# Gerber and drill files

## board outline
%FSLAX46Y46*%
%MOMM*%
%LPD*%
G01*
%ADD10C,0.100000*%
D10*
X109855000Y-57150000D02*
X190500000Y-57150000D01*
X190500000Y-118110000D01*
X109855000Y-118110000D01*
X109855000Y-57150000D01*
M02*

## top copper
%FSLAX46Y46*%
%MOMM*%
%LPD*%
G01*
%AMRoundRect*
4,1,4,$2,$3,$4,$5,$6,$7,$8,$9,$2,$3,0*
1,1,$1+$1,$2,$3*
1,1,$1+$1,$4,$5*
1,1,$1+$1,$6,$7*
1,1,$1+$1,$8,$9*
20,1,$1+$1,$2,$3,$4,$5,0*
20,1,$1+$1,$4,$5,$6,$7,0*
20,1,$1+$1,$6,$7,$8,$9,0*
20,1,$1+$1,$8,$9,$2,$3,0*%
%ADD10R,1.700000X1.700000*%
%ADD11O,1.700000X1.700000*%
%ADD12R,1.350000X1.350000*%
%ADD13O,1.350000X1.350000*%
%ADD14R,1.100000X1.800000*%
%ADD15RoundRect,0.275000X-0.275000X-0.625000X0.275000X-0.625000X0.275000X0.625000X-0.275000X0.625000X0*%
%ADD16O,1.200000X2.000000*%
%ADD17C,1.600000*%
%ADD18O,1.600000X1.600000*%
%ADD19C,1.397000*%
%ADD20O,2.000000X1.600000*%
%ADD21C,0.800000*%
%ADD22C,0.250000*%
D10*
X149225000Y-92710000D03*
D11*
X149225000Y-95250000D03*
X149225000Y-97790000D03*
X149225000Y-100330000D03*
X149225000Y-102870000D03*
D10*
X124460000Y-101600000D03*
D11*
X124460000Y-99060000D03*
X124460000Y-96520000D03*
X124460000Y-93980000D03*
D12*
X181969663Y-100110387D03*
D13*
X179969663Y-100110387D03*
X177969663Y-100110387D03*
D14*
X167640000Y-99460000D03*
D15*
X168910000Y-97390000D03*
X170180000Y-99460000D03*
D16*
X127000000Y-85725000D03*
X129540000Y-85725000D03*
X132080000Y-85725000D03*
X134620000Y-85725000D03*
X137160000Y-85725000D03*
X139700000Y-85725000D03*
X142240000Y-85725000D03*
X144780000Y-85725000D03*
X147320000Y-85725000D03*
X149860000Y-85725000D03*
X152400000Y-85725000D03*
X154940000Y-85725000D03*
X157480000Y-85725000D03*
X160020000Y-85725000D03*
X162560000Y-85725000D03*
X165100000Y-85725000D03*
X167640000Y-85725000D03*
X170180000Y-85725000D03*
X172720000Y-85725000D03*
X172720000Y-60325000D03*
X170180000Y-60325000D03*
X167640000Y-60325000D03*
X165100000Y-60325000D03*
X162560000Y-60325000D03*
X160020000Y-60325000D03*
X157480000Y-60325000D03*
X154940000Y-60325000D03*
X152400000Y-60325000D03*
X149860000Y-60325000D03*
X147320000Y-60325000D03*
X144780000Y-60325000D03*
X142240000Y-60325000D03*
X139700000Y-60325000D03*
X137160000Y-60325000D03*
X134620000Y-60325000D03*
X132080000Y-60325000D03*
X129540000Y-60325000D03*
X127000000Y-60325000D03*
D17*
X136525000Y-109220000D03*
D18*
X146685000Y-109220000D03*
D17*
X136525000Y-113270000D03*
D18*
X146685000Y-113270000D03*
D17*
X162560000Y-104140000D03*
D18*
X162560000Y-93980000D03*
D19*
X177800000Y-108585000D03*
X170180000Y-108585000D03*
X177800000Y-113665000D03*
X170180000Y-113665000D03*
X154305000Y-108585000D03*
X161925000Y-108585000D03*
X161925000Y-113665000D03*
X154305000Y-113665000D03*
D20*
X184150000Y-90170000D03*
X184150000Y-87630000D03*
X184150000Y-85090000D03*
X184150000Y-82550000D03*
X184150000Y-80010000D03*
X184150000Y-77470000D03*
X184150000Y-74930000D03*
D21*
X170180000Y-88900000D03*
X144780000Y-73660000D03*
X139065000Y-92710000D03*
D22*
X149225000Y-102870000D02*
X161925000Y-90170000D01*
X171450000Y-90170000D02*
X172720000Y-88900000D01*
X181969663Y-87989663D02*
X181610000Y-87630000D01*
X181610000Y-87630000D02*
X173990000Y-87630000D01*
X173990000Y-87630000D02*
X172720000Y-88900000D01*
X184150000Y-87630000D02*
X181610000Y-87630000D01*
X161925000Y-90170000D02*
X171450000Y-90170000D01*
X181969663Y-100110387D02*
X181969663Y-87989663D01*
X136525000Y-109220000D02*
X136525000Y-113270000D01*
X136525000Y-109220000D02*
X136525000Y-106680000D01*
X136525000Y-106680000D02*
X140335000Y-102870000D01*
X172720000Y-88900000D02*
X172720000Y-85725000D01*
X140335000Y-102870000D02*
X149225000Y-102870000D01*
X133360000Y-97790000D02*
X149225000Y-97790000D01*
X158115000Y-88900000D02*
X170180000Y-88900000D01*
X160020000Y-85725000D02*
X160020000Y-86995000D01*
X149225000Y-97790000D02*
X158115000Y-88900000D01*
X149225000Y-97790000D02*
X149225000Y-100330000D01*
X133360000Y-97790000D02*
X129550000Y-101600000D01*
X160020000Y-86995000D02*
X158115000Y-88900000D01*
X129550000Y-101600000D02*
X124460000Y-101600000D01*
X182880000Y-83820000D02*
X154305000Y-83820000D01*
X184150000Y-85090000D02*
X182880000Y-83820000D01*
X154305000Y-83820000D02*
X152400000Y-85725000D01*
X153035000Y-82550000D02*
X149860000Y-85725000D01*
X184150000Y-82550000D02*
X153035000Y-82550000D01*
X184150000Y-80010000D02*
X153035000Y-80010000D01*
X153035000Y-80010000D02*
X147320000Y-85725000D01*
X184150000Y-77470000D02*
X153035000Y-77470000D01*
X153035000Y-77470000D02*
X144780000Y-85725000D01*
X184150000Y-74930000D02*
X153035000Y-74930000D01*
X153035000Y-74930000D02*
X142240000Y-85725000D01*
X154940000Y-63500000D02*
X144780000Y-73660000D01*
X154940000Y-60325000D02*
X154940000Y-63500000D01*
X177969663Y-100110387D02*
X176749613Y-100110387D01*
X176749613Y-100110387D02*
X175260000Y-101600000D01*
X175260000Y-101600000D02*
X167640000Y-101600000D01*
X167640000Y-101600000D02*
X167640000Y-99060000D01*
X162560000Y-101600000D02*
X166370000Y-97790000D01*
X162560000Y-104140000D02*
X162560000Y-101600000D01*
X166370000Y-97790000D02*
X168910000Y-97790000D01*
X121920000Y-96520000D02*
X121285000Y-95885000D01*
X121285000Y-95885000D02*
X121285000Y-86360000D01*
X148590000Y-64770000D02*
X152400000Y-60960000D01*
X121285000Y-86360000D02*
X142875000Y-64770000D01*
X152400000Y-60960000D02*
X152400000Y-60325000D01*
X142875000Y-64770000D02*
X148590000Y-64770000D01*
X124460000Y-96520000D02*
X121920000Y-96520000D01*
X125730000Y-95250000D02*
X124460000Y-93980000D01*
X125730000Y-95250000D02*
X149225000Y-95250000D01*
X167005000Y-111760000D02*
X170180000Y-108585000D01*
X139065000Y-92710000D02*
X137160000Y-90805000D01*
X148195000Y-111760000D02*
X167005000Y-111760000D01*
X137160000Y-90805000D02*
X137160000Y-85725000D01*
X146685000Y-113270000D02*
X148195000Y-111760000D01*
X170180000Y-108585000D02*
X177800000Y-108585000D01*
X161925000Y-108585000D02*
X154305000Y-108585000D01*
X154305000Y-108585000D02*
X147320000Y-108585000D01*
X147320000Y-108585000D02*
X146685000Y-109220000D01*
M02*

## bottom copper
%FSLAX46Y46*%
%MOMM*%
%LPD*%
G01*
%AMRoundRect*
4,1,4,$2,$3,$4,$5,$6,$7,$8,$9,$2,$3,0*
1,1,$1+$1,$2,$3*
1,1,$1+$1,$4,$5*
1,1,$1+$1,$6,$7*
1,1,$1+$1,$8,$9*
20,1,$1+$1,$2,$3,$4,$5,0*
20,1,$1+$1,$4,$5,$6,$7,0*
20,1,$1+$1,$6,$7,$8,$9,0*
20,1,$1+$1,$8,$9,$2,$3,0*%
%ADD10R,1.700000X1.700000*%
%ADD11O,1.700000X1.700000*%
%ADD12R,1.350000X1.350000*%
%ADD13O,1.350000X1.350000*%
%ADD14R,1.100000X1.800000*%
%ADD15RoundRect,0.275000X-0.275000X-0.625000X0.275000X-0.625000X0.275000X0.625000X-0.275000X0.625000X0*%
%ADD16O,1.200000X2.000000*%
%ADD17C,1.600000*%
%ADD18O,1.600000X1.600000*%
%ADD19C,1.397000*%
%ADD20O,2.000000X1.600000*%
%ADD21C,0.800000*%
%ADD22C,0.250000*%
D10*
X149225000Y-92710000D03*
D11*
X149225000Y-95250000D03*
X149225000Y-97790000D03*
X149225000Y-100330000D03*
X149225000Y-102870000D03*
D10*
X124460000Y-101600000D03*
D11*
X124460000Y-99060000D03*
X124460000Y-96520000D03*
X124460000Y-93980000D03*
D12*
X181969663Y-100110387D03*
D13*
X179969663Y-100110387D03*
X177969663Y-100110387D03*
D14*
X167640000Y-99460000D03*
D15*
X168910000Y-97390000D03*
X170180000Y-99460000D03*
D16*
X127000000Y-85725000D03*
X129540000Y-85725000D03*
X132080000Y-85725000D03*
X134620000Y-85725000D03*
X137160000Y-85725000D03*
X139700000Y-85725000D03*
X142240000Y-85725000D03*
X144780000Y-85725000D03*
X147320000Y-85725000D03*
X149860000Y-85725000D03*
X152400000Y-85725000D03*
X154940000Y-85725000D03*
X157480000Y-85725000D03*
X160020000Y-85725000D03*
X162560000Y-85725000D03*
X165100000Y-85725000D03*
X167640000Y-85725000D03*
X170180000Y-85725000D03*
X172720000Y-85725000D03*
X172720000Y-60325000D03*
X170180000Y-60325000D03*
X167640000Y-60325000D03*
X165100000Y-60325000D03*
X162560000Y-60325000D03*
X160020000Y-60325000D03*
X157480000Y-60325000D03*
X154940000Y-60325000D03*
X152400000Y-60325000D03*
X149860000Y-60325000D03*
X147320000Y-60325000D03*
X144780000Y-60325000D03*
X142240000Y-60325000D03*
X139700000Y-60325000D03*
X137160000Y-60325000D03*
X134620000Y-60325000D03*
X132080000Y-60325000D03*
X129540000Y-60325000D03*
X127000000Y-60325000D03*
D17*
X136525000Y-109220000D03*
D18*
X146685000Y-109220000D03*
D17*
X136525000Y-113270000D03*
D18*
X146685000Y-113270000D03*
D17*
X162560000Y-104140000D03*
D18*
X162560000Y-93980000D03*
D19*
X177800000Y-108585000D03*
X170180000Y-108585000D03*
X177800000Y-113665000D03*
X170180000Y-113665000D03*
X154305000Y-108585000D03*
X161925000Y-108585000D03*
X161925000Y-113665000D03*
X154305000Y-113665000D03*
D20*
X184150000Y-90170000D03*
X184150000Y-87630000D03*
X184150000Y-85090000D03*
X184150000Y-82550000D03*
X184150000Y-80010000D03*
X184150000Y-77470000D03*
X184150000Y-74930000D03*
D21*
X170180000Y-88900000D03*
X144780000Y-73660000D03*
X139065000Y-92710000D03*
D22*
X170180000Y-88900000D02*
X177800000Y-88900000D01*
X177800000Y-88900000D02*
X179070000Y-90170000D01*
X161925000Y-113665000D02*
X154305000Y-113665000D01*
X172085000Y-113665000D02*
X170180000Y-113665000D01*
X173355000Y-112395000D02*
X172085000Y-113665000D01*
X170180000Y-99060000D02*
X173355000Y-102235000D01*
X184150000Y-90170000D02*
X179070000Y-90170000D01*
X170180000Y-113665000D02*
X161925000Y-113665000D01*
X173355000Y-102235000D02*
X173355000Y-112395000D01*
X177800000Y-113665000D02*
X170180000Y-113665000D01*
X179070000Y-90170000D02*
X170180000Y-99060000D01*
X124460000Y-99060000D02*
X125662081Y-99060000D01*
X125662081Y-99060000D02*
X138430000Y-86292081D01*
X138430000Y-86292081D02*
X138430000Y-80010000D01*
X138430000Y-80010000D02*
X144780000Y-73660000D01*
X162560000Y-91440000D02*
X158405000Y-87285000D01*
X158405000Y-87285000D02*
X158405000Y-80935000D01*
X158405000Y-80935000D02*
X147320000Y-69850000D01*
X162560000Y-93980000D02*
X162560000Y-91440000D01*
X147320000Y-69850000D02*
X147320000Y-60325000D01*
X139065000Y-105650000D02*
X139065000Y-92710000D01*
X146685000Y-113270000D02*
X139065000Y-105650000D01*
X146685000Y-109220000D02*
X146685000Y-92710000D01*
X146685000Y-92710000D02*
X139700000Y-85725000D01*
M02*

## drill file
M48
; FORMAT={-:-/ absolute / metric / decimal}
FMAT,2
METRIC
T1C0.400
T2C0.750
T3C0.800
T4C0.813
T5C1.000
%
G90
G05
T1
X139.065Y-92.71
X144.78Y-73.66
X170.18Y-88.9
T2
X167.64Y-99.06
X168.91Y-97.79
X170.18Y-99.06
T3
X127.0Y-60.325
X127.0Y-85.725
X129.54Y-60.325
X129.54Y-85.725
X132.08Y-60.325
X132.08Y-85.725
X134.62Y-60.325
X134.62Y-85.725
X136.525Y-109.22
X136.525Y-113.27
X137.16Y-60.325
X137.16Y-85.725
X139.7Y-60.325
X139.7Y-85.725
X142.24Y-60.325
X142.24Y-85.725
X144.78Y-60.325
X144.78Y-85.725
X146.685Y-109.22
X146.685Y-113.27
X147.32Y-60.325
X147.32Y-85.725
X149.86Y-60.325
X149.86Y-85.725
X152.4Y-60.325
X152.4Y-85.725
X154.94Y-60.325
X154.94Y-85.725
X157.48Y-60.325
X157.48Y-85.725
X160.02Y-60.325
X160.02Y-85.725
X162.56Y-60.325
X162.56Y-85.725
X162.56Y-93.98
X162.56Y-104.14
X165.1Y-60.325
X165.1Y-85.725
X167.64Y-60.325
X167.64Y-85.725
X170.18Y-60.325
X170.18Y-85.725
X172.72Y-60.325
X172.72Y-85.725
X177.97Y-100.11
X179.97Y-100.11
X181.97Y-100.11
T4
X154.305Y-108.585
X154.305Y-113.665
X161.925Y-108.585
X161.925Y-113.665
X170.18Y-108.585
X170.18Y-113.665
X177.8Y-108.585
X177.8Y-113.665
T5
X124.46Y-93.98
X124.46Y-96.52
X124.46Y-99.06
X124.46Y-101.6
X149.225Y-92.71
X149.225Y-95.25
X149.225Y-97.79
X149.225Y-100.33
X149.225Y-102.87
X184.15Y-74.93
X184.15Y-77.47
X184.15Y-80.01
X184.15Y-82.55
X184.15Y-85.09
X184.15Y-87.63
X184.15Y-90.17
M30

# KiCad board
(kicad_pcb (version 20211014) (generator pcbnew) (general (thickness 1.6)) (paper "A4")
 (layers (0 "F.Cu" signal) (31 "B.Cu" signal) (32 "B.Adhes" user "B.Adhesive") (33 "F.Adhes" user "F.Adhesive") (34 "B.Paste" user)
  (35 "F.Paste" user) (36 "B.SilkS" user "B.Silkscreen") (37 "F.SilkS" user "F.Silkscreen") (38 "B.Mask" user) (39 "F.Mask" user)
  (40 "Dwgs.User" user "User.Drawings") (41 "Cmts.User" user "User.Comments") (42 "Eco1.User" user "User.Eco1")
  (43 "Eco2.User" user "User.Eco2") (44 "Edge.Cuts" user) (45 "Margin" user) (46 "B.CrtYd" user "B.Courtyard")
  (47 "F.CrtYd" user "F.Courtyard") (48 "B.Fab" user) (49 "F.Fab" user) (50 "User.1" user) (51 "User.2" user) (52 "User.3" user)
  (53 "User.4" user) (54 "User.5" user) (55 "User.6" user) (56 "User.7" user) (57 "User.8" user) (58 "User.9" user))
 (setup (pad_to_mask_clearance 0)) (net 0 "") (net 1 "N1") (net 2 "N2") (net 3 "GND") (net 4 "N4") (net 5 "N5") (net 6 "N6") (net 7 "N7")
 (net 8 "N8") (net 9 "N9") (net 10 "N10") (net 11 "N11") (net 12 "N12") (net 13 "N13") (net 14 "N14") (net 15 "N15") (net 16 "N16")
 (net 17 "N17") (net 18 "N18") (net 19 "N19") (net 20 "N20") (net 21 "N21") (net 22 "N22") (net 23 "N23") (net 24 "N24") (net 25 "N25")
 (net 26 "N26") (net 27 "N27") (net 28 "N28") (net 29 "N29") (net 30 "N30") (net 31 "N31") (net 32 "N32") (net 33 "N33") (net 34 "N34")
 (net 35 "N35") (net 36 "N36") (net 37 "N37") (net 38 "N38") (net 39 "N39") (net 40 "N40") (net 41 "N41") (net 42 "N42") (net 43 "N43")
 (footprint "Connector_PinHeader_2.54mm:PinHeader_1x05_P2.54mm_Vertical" (layer "F.Cu") (at 149.225 92.71)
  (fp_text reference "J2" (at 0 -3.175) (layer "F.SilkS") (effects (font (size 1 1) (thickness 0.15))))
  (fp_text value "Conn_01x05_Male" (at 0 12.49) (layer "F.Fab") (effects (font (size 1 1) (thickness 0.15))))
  (pad "1" thru_hole rect (at 0 0) (size 1.7 1.7) (drill 1) (layers *.Cu *.Mask) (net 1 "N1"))
  (pad "2" thru_hole oval (at 0 2.54) (size 1.7 1.7) (drill 1) (layers *.Cu *.Mask) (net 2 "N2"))
  (pad "3" thru_hole oval (at 0 5.08) (size 1.7 1.7) (drill 1) (layers *.Cu *.Mask) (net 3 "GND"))
  (pad "4" thru_hole oval (at 0 7.62) (size 1.7 1.7) (drill 1) (layers *.Cu *.Mask) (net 3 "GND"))
  (pad "5" thru_hole oval (at 0 10.16) (size 1.7 1.7) (drill 1) (layers *.Cu *.Mask) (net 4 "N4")))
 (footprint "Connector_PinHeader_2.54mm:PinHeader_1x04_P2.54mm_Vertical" (layer "F.Cu") (at 124.46 101.6 180)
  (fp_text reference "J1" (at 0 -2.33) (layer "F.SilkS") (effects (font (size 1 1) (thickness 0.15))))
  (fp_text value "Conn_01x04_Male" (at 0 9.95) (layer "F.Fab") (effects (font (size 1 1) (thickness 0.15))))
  (pad "1" thru_hole rect (at 0 0 180) (size 1.7 1.7) (drill 1) (layers *.Cu *.Mask) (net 3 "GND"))
  (pad "2" thru_hole oval (at 0 2.54 180) (size 1.7 1.7) (drill 1) (layers *.Cu *.Mask) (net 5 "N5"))
  (pad "3" thru_hole oval (at 0 5.08 180) (size 1.7 1.7) (drill 1) (layers *.Cu *.Mask) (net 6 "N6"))
  (pad "4" thru_hole oval (at 0 7.62 180) (size 1.7 1.7) (drill 1) (layers *.Cu *.Mask) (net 2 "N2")))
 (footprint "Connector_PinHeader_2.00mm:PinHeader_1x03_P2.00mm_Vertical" (layer "F.Cu") (at 181.969663 100.110387 -90)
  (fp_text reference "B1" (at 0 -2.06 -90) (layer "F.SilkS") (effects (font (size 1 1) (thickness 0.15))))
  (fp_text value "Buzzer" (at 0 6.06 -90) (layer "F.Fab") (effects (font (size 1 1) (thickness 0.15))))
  (pad "1" thru_hole rect (at 0 0 270) (size 1.35 1.35) (drill 0.8) (layers *.Cu *.Mask) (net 4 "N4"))
  (pad "2" thru_hole oval (at 0 2 270) (size 1.35 1.35) (drill 0.8) (layers *.Cu *.Mask) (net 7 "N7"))
  (pad "3" thru_hole oval (at 0 4 270) (size 1.35 1.35) (drill 0.8) (layers *.Cu *.Mask) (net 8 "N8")))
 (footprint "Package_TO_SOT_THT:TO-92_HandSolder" (layer "F.Cu") (at 167.64 99.06)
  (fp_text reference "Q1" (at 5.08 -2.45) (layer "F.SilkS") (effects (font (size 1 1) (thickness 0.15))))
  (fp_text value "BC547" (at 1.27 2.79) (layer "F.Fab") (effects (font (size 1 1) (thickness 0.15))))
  (pad "1" thru_hole rect (at 0 0) (size 1.1 1.8) (drill 0.75 (offset 0 0.4)) (layers *.Cu *.Mask) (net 8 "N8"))
  (pad "2" thru_hole roundrect (at 1.27 -1.27) (size 1.1 1.8) (drill 0.75 (offset 0 -0.4)) (layers *.Cu *.Mask) (roundrect_rratio 0.25)
   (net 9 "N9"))
  (pad "3" thru_hole roundrect (at 2.54 0) (size 1.1 1.8) (drill 0.75 (offset 0 0.4)) (layers *.Cu *.Mask) (roundrect_rratio 0.25)
   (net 3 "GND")))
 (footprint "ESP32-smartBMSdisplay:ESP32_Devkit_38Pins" (layer "F.Cu") (at 149.86 73.025)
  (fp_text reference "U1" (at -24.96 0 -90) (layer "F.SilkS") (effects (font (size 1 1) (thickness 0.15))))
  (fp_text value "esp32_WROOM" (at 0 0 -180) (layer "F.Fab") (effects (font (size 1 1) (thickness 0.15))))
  (pad "1" thru_hole oval (at -22.86 12.7) (size 1.2 2) (drill 0.8) (layers *.Cu *.Mask) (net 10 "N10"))
  (pad "2" thru_hole oval (at -20.32 12.7) (size 1.2 2) (drill 0.8) (layers *.Cu *.Mask) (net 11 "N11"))
  (pad "3" thru_hole oval (at -17.78 12.7) (size 1.2 2) (drill 0.8) (layers *.Cu *.Mask) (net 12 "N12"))
  (pad "4" thru_hole oval (at -15.24 12.7) (size 1.2 2) (drill 0.8) (layers *.Cu *.Mask) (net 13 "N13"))
  (pad "5" thru_hole oval (at -12.7 12.7) (size 1.2 2) (drill 0.8) (layers *.Cu *.Mask) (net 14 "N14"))
  (pad "6" thru_hole oval (at -10.16 12.7) (size 1.2 2) (drill 0.8) (layers *.Cu *.Mask) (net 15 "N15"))
  (pad "7" thru_hole oval (at -7.62 12.7) (size 1.2 2) (drill 0.8) (layers *.Cu *.Mask) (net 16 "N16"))
  (pad "8" thru_hole oval (at -5.08 12.7) (size 1.2 2) (drill 0.8) (layers *.Cu *.Mask) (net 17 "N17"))
  (pad "9" thru_hole oval (at -2.54 12.7) (size 1.2 2) (drill 0.8) (layers *.Cu *.Mask) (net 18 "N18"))
  (pad "10" thru_hole oval (at 0 12.7) (size 1.2 2) (drill 0.8) (layers *.Cu *.Mask) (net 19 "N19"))
  (pad "11" thru_hole oval (at 2.54 12.7) (size 1.2 2) (drill 0.8) (layers *.Cu *.Mask) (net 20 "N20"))
  (pad "12" thru_hole oval (at 5.08 12.7) (size 1.2 2) (drill 0.8) (layers *.Cu *.Mask) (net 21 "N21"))
  (pad "13" thru_hole oval (at 7.62 12.7) (size 1.2 2) (drill 0.8) (layers *.Cu *.Mask) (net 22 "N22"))
  (pad "14" thru_hole oval (at 10.16 12.7) (size 1.2 2) (drill 0.8) (layers *.Cu *.Mask) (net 3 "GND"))
  (pad "15" thru_hole oval (at 12.7 12.7) (size 1.2 2) (drill 0.8) (layers *.Cu *.Mask) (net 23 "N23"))
  (pad "16" thru_hole oval (at 15.24 12.7) (size 1.2 2) (drill 0.8) (layers *.Cu *.Mask) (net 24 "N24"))
  (pad "17" thru_hole oval (at 17.78 12.7) (size 1.2 2) (drill 0.8) (layers *.Cu *.Mask) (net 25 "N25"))
  (pad "18" thru_hole oval (at 20.32 12.7) (size 1.2 2) (drill 0.8) (layers *.Cu *.Mask) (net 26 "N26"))
  (pad "19" thru_hole oval (at 22.86 12.7) (size 1.2 2) (drill 0.8) (layers *.Cu *.Mask) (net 4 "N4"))
  (pad "20" thru_hole oval (at 22.86 -12.7) (size 1.2 2) (drill 0.8) (layers *.Cu *.Mask) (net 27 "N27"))
  (pad "21" thru_hole oval (at 20.32 -12.7) (size 1.2 2) (drill 0.8) (layers *.Cu *.Mask) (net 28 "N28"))
  (pad "22" thru_hole oval (at 17.78 -12.7) (size 1.2 2) (drill 0.8) (layers *.Cu *.Mask) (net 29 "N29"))
  (pad "23" thru_hole oval (at 15.24 -12.7) (size 1.2 2) (drill 0.8) (layers *.Cu *.Mask) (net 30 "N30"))
  (pad "24" thru_hole oval (at 12.7 -12.7) (size 1.2 2) (drill 0.8) (layers *.Cu *.Mask) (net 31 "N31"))
  (pad "25" thru_hole oval (at 10.16 -12.7) (size 1.2 2) (drill 0.8) (layers *.Cu *.Mask) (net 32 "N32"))
  (pad "26" thru_hole oval (at 7.62 -12.7) (size 1.2 2) (drill 0.8) (layers *.Cu *.Mask) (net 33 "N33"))
  (pad "27" thru_hole oval (at 5.08 -12.7) (size 1.2 2) (drill 0.8) (layers *.Cu *.Mask) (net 5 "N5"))
  (pad "28" thru_hole oval (at 2.54 -12.7) (size 1.2 2) (drill 0.8) (layers *.Cu *.Mask) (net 6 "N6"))
  (pad "29" thru_hole oval (at 0 -12.7) (size 1.2 2) (drill 0.8) (layers *.Cu *.Mask) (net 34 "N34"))
  (pad "30" thru_hole oval (at -2.54 -12.7) (size 1.2 2) (drill 0.8) (layers *.Cu *.Mask) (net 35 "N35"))
  (pad "31" thru_hole oval (at -5.08 -12.7) (size 1.2 2) (drill 0.8) (layers *.Cu *.Mask) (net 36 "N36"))
  (pad "32" thru_hole oval (at -7.62 -12.7) (size 1.2 2) (drill 0.8) (layers *.Cu *.Mask) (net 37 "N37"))
  (pad "33" thru_hole oval (at -10.16 -12.7) (size 1.2 2) (drill 0.8) (layers *.Cu *.Mask) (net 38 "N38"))
  (pad "34" thru_hole oval (at -12.7 -12.7) (size 1.2 2) (drill 0.8) (layers *.Cu *.Mask) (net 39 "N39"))
  (pad "35" thru_hole oval (at -15.24 -12.7) (size 1.2 2) (drill 0.8) (layers *.Cu *.Mask) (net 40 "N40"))
  (pad "36" thru_hole oval (at -17.78 -12.7) (size 1.2 2) (drill 0.8) (layers *.Cu *.Mask) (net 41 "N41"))
  (pad "37" thru_hole oval (at -20.32 -12.7) (size 1.2 2) (drill 0.8) (layers *.Cu *.Mask) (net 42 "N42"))
  (pad "38" thru_hole oval (at -22.86 -12.7) (size 1.2 2) (drill 0.8) (layers *.Cu *.Mask) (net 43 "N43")))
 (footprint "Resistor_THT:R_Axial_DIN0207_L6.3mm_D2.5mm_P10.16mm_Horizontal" (layer "F.Cu") (at 136.525 109.22)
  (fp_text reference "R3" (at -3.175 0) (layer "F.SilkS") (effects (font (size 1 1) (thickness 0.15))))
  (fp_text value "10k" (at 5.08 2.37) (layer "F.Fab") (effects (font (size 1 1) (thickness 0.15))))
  (pad "1" thru_hole circle (at 0 0) (size 1.6 1.6) (drill 0.8) (layers *.Cu *.Mask) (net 4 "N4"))
  (pad "2" thru_hole oval (at 10.16 0) (size 1.6 1.6) (drill 0.8) (layers *.Cu *.Mask) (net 15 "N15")))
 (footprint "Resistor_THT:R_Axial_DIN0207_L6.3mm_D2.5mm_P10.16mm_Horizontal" (layer "F.Cu") (at 136.525 113.27)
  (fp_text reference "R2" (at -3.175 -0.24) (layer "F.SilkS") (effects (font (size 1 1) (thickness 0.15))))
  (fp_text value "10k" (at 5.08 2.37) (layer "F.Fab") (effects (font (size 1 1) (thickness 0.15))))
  (pad "1" thru_hole circle (at 0 0) (size 1.6 1.6) (drill 0.8) (layers *.Cu *.Mask) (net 4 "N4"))
  (pad "2" thru_hole oval (at 10.16 0) (size 1.6 1.6) (drill 0.8) (layers *.Cu *.Mask) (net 14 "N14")))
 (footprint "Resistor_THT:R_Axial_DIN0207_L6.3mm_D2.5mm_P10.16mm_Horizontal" (layer "F.Cu") (at 162.56 104.14 90)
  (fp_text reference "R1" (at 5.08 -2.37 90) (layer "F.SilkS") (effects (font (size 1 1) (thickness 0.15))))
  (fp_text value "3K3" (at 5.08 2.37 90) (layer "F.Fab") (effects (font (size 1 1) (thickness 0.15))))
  (pad "1" thru_hole circle (at 0 0 90) (size 1.6 1.6) (drill 0.8) (layers *.Cu *.Mask) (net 9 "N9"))
  (pad "2" thru_hole oval (at 10.16 0 90) (size 1.6 1.6) (drill 0.8) (layers *.Cu *.Mask) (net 35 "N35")))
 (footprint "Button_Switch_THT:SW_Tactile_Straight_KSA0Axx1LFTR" (layer "B.Cu") (at 177.8 108.585 180)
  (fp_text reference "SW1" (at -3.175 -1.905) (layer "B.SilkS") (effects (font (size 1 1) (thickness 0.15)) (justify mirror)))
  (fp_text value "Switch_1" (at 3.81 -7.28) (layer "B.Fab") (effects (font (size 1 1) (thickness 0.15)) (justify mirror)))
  (pad "1" thru_hole circle (at 0 0 180) (size 1.397 1.397) (drill 0.8128) (layers *.Cu *.Mask) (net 14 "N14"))
  (pad "1" thru_hole circle (at 7.62 0 180) (size 1.397 1.397) (drill 0.8128) (layers *.Cu *.Mask) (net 14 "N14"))
  (pad "2" thru_hole circle (at 0 -5.08 180) (size 1.397 1.397) (drill 0.8128) (layers *.Cu *.Mask) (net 3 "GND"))
  (pad "2" thru_hole circle (at 7.62 -5.08 180) (size 1.397 1.397) (drill 0.8128) (layers *.Cu *.Mask) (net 3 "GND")))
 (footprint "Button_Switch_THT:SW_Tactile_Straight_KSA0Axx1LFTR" (layer "B.Cu") (at 161.925 108.585 180)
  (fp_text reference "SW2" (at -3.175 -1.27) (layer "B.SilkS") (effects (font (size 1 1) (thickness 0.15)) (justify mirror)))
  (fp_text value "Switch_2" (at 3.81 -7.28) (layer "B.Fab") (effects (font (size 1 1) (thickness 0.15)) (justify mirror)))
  (pad "1" thru_hole circle (at 7.62 0 180) (size 1.397 1.397) (drill 0.8128) (layers *.Cu *.Mask) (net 15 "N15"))
  (pad "1" thru_hole circle (at 0 0 180) (size 1.397 1.397) (drill 0.8128) (layers *.Cu *.Mask) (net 15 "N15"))
  (pad "2" thru_hole circle (at 0 -5.08 180) (size 1.397 1.397) (drill 0.8128) (layers *.Cu *.Mask) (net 3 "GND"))
  (pad "2" thru_hole circle (at 7.62 -5.08 180) (size 1.397 1.397) (drill 0.8128) (layers *.Cu *.Mask) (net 3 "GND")))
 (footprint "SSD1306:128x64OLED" (layer "B.Cu") (at 171.45 82.55 180)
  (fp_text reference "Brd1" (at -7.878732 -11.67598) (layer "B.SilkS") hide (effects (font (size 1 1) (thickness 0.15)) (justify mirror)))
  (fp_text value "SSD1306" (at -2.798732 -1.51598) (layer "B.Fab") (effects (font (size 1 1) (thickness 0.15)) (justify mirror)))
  (pad "1" thru_hole oval (at -12.7 -7.62) (size 2 1.6) (drill 1) (layers *.Cu *.Mask) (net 3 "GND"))
  (pad "2" thru_hole oval (at -12.7 -5.08) (size 2 1.6) (drill 1) (layers *.Cu *.Mask) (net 4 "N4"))
  (pad "3" thru_hole oval (at -12.7 -2.54) (size 2 1.6) (drill 1) (layers *.Cu *.Mask) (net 20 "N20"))
  (pad "4" thru_hole oval (at -12.7 0) (size 2 1.6) (drill 1) (layers *.Cu *.Mask) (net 19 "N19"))
  (pad "5" thru_hole oval (at -12.7 2.54) (size 2 1.6) (drill 1) (layers *.Cu *.Mask) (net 18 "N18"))
  (pad "6" thru_hole oval (at -12.7 5.08) (size 2 1.6) (drill 1) (layers *.Cu *.Mask) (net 17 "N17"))
  (pad "7" thru_hole oval (at -12.7 7.62) (size 2 1.6) (drill 1) (layers *.Cu *.Mask) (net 16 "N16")))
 (gr_rect (start 109.855 118.11) (end 190.5 57.15) (layer "Edge.Cuts") (width 0.1) (fill none))
 (segment (start 149.225 102.87) (end 161.925 90.17) (width 0.25) (layer "F.Cu") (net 4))
 (segment (start 171.45 90.17) (end 172.72 88.9) (width 0.25) (layer "F.Cu") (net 4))
 (segment (start 181.969663 87.989663) (end 181.61 87.63) (width 0.25) (layer "F.Cu") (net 4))
 (segment (start 181.61 87.63) (end 173.99 87.63) (width 0.25) (layer "F.Cu") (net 4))
 (segment (start 173.99 87.63) (end 172.72 88.9) (width 0.25) (layer "F.Cu") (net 4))
 (segment (start 184.15 87.63) (end 181.61 87.63) (width 0.25) (layer "F.Cu") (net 4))
 (segment (start 161.925 90.17) (end 171.45 90.17) (width 0.25) (layer "F.Cu") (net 4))
 (segment (start 181.969663 100.110387) (end 181.969663 87.989663) (width 0.25) (layer "F.Cu") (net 4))
 (segment (start 136.525 109.22) (end 136.525 113.27) (width 0.25) (layer "F.Cu") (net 4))
 (segment (start 136.525 109.22) (end 136.525 106.68) (width 0.25) (layer "F.Cu") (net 4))
 (segment (start 136.525 106.68) (end 140.335 102.87) (width 0.25) (layer "F.Cu") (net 4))
 (segment (start 172.72 88.9) (end 172.72 85.725) (width 0.25) (layer "F.Cu") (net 4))
 (segment (start 140.335 102.87) (end 149.225 102.87) (width 0.25) (layer "F.Cu") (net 4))
 (segment (start 133.36 97.79) (end 149.225 97.79) (width 0.25) (layer "F.Cu") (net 3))
 (segment (start 158.115 88.9) (end 170.18 88.9) (width 0.25) (layer "F.Cu") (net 3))
 (segment (start 160.02 85.725) (end 160.02 86.995) (width 0.25) (layer "F.Cu") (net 3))
 (segment (start 149.225 97.79) (end 158.115 88.9) (width 0.25) (layer "F.Cu") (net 3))
 (segment (start 149.225 97.79) (end 149.225 100.33) (width 0.25) (layer "F.Cu") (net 3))
 (segment (start 133.36 97.79) (end 129.55 101.6) (width 0.25) (layer "F.Cu") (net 3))
 (segment (start 160.02 86.995) (end 158.115 88.9) (width 0.25) (layer "F.Cu") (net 3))
 (segment (start 129.55 101.6) (end 124.46 101.6) (width 0.25) (layer "F.Cu") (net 3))
 (via (at 170.18 88.9) (size 0.8) (drill 0.4) (layers "F.Cu" "B.Cu") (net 3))
 (segment (start 170.18 88.9) (end 177.8 88.9) (width 0.25) (layer "B.Cu") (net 3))
 (segment (start 177.8 88.9) (end 179.07 90.17) (width 0.25) (layer "B.Cu") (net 3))
 (segment (start 161.925 113.665) (end 154.305 113.665) (width 0.25) (layer "B.Cu") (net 3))
 (segment (start 172.085 113.665) (end 170.18 113.665) (width 0.25) (layer "B.Cu") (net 3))
 (segment (start 173.355 112.395) (end 172.085 113.665) (width 0.25) (layer "B.Cu") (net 3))
 (segment (start 170.18 99.06) (end 173.355 102.235) (width 0.25) (layer "B.Cu") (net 3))
 (segment (start 184.15 90.17) (end 179.07 90.17) (width 0.25) (layer "B.Cu") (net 3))
 (segment (start 170.18 113.665) (end 161.925 113.665) (width 0.25) (layer "B.Cu") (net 3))
 (segment (start 173.355 102.235) (end 173.355 112.395) (width 0.25) (layer "B.Cu") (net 3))
 (segment (start 177.8 113.665) (end 170.18 113.665) (width 0.25) (layer "B.Cu") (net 3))
 (segment (start 179.07 90.17) (end 170.18 99.06) (width 0.25) (layer "B.Cu") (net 3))
 (segment (start 182.88 83.82) (end 154.305 83.82) (width 0.25) (layer "F.Cu") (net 20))
 (segment (start 184.15 85.09) (end 182.88 83.82) (width 0.25) (layer "F.Cu") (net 20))
 (segment (start 154.305 83.82) (end 152.4 85.725) (width 0.25) (layer "F.Cu") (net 20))
 (segment (start 153.035 82.55) (end 149.86 85.725) (width 0.25) (layer "F.Cu") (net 19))
 (segment (start 184.15 82.55) (end 153.035 82.55) (width 0.25) (layer "F.Cu") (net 19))
 (segment (start 184.15 80.01) (end 153.035 80.01) (width 0.25) (layer "F.Cu") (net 18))
 (segment (start 153.035 80.01) (end 147.32 85.725) (width 0.25) (layer "F.Cu") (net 18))
 (segment (start 184.15 77.47) (end 153.035 77.47) (width 0.25) (layer "F.Cu") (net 17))
 (segment (start 153.035 77.47) (end 144.78 85.725) (width 0.25) (layer "F.Cu") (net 17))
 (segment (start 184.15 74.93) (end 153.035 74.93) (width 0.25) (layer "F.Cu") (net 16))
 (segment (start 153.035 74.93) (end 142.24 85.725) (width 0.25) (layer "F.Cu") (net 16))
 (segment (start 154.94 63.5) (end 144.78 73.66) (width 0.25) (layer "F.Cu") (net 5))
 (segment (start 154.94 60.325) (end 154.94 63.5) (width 0.25) (layer "F.Cu") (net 5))
 (via (at 144.78 73.66) (size 0.8) (drill 0.4) (layers "F.Cu" "B.Cu") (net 5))
 (segment (start 124.46 99.06) (end 125.662081 99.06) (width 0.25) (layer "B.Cu") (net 5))
 (segment (start 125.662081 99.06) (end 138.43 86.292081) (width 0.25) (layer "B.Cu") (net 5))
 (segment (start 138.43 86.292081) (end 138.43 80.01) (width 0.25) (layer "B.Cu") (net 5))
 (segment (start 138.43 80.01) (end 144.78 73.66) (width 0.25) (layer "B.Cu") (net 5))
 (segment (start 177.969663 100.110387) (end 176.749613 100.110387) (width 0.25) (layer "F.Cu") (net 8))
 (segment (start 176.749613 100.110387) (end 175.26 101.6) (width 0.25) (layer "F.Cu") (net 8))
 (segment (start 175.26 101.6) (end 167.64 101.6) (width 0.25) (layer "F.Cu") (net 8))
 (segment (start 167.64 101.6) (end 167.64 99.06) (width 0.25) (layer "F.Cu") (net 8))
 (segment (start 162.56 101.6) (end 166.37 97.79) (width 0.25) (layer "F.Cu") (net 9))
 (segment (start 162.56 104.14) (end 162.56 101.6) (width 0.25) (layer "F.Cu") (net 9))
 (segment (start 166.37 97.79) (end 168.91 97.79) (width 0.25) (layer "F.Cu") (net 9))
 (segment (start 121.92 96.52) (end 121.285 95.885) (width 0.25) (layer "F.Cu") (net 6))
 (segment (start 121.285 95.885) (end 121.285 86.36) (width 0.25) (layer "F.Cu") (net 6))
 (segment (start 148.59 64.77) (end 152.4 60.96) (width 0.25) (layer "F.Cu") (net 6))
 (segment (start 121.285 86.36) (end 142.875 64.77) (width 0.25) (layer "F.Cu") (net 6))
 (segment (start 152.4 60.96) (end 152.4 60.325) (width 0.25) (layer "F.Cu") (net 6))
 (segment (start 142.875 64.77) (end 148.59 64.77) (width 0.25) (layer "F.Cu") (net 6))
 (segment (start 124.46 96.52) (end 121.92 96.52) (width 0.25) (layer "F.Cu") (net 6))
 (segment (start 162.56 91.44) (end 158.405 87.285) (width 0.25) (layer "B.Cu") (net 35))
 (segment (start 158.405 87.285) (end 158.405 80.935) (width 0.25) (layer "B.Cu") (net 35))
 (segment (start 158.405 80.935) (end 147.32 69.85) (width 0.25) (layer "B.Cu") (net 35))
 (segment (start 162.56 93.98) (end 162.56 91.44) (width 0.25) (layer "B.Cu") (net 35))
 (segment (start 147.32 69.85) (end 147.32 60.325) (width 0.25) (layer "B.Cu") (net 35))
 (segment (start 125.73 95.25) (end 124.46 93.98) (width 0.25) (layer "F.Cu") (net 2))
 (segment (start 125.73 95.25) (end 149.225 95.25) (width 0.25) (layer "F.Cu") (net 2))
 (segment (start 167.005 111.76) (end 170.18 108.585) (width 0.25) (layer "F.Cu") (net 14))
 (segment (start 139.065 92.71) (end 137.16 90.805) (width 0.25) (layer "F.Cu") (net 14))
 (segment (start 148.195 111.76) (end 167.005 111.76) (width 0.25) (layer "F.Cu") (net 14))
 (segment (start 137.16 90.805) (end 137.16 85.725) (width 0.25) (layer "F.Cu") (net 14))
 (segment (start 146.685 113.27) (end 148.195 111.76) (width 0.25) (layer "F.Cu") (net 14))
 (segment (start 170.18 108.585) (end 177.8 108.585) (width 0.25) (layer "F.Cu") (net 14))
 (via (at 139.065 92.71) (size 0.8) (drill 0.4) (layers "F.Cu" "B.Cu") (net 14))
 (segment (start 139.065 105.65) (end 139.065 92.71) (width 0.25) (layer "B.Cu") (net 14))
 (segment (start 146.685 113.27) (end 139.065 105.65) (width 0.25) (layer "B.Cu") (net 14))
 (segment (start 161.925 108.585) (end 154.305 108.585) (width 0.25) (layer "F.Cu") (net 15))
 (segment (start 154.305 108.585) (end 147.32 108.585) (width 0.25) (layer "F.Cu") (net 15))
 (segment (start 147.32 108.585) (end 146.685 109.22) (width 0.25) (layer "F.Cu") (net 15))
 (segment (start 146.685 109.22) (end 146.685 92.71) (width 0.25) (layer "B.Cu") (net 15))
 (segment (start 146.685 92.71) (end 139.7 85.725) (width 0.25) (layer "B.Cu") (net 15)))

